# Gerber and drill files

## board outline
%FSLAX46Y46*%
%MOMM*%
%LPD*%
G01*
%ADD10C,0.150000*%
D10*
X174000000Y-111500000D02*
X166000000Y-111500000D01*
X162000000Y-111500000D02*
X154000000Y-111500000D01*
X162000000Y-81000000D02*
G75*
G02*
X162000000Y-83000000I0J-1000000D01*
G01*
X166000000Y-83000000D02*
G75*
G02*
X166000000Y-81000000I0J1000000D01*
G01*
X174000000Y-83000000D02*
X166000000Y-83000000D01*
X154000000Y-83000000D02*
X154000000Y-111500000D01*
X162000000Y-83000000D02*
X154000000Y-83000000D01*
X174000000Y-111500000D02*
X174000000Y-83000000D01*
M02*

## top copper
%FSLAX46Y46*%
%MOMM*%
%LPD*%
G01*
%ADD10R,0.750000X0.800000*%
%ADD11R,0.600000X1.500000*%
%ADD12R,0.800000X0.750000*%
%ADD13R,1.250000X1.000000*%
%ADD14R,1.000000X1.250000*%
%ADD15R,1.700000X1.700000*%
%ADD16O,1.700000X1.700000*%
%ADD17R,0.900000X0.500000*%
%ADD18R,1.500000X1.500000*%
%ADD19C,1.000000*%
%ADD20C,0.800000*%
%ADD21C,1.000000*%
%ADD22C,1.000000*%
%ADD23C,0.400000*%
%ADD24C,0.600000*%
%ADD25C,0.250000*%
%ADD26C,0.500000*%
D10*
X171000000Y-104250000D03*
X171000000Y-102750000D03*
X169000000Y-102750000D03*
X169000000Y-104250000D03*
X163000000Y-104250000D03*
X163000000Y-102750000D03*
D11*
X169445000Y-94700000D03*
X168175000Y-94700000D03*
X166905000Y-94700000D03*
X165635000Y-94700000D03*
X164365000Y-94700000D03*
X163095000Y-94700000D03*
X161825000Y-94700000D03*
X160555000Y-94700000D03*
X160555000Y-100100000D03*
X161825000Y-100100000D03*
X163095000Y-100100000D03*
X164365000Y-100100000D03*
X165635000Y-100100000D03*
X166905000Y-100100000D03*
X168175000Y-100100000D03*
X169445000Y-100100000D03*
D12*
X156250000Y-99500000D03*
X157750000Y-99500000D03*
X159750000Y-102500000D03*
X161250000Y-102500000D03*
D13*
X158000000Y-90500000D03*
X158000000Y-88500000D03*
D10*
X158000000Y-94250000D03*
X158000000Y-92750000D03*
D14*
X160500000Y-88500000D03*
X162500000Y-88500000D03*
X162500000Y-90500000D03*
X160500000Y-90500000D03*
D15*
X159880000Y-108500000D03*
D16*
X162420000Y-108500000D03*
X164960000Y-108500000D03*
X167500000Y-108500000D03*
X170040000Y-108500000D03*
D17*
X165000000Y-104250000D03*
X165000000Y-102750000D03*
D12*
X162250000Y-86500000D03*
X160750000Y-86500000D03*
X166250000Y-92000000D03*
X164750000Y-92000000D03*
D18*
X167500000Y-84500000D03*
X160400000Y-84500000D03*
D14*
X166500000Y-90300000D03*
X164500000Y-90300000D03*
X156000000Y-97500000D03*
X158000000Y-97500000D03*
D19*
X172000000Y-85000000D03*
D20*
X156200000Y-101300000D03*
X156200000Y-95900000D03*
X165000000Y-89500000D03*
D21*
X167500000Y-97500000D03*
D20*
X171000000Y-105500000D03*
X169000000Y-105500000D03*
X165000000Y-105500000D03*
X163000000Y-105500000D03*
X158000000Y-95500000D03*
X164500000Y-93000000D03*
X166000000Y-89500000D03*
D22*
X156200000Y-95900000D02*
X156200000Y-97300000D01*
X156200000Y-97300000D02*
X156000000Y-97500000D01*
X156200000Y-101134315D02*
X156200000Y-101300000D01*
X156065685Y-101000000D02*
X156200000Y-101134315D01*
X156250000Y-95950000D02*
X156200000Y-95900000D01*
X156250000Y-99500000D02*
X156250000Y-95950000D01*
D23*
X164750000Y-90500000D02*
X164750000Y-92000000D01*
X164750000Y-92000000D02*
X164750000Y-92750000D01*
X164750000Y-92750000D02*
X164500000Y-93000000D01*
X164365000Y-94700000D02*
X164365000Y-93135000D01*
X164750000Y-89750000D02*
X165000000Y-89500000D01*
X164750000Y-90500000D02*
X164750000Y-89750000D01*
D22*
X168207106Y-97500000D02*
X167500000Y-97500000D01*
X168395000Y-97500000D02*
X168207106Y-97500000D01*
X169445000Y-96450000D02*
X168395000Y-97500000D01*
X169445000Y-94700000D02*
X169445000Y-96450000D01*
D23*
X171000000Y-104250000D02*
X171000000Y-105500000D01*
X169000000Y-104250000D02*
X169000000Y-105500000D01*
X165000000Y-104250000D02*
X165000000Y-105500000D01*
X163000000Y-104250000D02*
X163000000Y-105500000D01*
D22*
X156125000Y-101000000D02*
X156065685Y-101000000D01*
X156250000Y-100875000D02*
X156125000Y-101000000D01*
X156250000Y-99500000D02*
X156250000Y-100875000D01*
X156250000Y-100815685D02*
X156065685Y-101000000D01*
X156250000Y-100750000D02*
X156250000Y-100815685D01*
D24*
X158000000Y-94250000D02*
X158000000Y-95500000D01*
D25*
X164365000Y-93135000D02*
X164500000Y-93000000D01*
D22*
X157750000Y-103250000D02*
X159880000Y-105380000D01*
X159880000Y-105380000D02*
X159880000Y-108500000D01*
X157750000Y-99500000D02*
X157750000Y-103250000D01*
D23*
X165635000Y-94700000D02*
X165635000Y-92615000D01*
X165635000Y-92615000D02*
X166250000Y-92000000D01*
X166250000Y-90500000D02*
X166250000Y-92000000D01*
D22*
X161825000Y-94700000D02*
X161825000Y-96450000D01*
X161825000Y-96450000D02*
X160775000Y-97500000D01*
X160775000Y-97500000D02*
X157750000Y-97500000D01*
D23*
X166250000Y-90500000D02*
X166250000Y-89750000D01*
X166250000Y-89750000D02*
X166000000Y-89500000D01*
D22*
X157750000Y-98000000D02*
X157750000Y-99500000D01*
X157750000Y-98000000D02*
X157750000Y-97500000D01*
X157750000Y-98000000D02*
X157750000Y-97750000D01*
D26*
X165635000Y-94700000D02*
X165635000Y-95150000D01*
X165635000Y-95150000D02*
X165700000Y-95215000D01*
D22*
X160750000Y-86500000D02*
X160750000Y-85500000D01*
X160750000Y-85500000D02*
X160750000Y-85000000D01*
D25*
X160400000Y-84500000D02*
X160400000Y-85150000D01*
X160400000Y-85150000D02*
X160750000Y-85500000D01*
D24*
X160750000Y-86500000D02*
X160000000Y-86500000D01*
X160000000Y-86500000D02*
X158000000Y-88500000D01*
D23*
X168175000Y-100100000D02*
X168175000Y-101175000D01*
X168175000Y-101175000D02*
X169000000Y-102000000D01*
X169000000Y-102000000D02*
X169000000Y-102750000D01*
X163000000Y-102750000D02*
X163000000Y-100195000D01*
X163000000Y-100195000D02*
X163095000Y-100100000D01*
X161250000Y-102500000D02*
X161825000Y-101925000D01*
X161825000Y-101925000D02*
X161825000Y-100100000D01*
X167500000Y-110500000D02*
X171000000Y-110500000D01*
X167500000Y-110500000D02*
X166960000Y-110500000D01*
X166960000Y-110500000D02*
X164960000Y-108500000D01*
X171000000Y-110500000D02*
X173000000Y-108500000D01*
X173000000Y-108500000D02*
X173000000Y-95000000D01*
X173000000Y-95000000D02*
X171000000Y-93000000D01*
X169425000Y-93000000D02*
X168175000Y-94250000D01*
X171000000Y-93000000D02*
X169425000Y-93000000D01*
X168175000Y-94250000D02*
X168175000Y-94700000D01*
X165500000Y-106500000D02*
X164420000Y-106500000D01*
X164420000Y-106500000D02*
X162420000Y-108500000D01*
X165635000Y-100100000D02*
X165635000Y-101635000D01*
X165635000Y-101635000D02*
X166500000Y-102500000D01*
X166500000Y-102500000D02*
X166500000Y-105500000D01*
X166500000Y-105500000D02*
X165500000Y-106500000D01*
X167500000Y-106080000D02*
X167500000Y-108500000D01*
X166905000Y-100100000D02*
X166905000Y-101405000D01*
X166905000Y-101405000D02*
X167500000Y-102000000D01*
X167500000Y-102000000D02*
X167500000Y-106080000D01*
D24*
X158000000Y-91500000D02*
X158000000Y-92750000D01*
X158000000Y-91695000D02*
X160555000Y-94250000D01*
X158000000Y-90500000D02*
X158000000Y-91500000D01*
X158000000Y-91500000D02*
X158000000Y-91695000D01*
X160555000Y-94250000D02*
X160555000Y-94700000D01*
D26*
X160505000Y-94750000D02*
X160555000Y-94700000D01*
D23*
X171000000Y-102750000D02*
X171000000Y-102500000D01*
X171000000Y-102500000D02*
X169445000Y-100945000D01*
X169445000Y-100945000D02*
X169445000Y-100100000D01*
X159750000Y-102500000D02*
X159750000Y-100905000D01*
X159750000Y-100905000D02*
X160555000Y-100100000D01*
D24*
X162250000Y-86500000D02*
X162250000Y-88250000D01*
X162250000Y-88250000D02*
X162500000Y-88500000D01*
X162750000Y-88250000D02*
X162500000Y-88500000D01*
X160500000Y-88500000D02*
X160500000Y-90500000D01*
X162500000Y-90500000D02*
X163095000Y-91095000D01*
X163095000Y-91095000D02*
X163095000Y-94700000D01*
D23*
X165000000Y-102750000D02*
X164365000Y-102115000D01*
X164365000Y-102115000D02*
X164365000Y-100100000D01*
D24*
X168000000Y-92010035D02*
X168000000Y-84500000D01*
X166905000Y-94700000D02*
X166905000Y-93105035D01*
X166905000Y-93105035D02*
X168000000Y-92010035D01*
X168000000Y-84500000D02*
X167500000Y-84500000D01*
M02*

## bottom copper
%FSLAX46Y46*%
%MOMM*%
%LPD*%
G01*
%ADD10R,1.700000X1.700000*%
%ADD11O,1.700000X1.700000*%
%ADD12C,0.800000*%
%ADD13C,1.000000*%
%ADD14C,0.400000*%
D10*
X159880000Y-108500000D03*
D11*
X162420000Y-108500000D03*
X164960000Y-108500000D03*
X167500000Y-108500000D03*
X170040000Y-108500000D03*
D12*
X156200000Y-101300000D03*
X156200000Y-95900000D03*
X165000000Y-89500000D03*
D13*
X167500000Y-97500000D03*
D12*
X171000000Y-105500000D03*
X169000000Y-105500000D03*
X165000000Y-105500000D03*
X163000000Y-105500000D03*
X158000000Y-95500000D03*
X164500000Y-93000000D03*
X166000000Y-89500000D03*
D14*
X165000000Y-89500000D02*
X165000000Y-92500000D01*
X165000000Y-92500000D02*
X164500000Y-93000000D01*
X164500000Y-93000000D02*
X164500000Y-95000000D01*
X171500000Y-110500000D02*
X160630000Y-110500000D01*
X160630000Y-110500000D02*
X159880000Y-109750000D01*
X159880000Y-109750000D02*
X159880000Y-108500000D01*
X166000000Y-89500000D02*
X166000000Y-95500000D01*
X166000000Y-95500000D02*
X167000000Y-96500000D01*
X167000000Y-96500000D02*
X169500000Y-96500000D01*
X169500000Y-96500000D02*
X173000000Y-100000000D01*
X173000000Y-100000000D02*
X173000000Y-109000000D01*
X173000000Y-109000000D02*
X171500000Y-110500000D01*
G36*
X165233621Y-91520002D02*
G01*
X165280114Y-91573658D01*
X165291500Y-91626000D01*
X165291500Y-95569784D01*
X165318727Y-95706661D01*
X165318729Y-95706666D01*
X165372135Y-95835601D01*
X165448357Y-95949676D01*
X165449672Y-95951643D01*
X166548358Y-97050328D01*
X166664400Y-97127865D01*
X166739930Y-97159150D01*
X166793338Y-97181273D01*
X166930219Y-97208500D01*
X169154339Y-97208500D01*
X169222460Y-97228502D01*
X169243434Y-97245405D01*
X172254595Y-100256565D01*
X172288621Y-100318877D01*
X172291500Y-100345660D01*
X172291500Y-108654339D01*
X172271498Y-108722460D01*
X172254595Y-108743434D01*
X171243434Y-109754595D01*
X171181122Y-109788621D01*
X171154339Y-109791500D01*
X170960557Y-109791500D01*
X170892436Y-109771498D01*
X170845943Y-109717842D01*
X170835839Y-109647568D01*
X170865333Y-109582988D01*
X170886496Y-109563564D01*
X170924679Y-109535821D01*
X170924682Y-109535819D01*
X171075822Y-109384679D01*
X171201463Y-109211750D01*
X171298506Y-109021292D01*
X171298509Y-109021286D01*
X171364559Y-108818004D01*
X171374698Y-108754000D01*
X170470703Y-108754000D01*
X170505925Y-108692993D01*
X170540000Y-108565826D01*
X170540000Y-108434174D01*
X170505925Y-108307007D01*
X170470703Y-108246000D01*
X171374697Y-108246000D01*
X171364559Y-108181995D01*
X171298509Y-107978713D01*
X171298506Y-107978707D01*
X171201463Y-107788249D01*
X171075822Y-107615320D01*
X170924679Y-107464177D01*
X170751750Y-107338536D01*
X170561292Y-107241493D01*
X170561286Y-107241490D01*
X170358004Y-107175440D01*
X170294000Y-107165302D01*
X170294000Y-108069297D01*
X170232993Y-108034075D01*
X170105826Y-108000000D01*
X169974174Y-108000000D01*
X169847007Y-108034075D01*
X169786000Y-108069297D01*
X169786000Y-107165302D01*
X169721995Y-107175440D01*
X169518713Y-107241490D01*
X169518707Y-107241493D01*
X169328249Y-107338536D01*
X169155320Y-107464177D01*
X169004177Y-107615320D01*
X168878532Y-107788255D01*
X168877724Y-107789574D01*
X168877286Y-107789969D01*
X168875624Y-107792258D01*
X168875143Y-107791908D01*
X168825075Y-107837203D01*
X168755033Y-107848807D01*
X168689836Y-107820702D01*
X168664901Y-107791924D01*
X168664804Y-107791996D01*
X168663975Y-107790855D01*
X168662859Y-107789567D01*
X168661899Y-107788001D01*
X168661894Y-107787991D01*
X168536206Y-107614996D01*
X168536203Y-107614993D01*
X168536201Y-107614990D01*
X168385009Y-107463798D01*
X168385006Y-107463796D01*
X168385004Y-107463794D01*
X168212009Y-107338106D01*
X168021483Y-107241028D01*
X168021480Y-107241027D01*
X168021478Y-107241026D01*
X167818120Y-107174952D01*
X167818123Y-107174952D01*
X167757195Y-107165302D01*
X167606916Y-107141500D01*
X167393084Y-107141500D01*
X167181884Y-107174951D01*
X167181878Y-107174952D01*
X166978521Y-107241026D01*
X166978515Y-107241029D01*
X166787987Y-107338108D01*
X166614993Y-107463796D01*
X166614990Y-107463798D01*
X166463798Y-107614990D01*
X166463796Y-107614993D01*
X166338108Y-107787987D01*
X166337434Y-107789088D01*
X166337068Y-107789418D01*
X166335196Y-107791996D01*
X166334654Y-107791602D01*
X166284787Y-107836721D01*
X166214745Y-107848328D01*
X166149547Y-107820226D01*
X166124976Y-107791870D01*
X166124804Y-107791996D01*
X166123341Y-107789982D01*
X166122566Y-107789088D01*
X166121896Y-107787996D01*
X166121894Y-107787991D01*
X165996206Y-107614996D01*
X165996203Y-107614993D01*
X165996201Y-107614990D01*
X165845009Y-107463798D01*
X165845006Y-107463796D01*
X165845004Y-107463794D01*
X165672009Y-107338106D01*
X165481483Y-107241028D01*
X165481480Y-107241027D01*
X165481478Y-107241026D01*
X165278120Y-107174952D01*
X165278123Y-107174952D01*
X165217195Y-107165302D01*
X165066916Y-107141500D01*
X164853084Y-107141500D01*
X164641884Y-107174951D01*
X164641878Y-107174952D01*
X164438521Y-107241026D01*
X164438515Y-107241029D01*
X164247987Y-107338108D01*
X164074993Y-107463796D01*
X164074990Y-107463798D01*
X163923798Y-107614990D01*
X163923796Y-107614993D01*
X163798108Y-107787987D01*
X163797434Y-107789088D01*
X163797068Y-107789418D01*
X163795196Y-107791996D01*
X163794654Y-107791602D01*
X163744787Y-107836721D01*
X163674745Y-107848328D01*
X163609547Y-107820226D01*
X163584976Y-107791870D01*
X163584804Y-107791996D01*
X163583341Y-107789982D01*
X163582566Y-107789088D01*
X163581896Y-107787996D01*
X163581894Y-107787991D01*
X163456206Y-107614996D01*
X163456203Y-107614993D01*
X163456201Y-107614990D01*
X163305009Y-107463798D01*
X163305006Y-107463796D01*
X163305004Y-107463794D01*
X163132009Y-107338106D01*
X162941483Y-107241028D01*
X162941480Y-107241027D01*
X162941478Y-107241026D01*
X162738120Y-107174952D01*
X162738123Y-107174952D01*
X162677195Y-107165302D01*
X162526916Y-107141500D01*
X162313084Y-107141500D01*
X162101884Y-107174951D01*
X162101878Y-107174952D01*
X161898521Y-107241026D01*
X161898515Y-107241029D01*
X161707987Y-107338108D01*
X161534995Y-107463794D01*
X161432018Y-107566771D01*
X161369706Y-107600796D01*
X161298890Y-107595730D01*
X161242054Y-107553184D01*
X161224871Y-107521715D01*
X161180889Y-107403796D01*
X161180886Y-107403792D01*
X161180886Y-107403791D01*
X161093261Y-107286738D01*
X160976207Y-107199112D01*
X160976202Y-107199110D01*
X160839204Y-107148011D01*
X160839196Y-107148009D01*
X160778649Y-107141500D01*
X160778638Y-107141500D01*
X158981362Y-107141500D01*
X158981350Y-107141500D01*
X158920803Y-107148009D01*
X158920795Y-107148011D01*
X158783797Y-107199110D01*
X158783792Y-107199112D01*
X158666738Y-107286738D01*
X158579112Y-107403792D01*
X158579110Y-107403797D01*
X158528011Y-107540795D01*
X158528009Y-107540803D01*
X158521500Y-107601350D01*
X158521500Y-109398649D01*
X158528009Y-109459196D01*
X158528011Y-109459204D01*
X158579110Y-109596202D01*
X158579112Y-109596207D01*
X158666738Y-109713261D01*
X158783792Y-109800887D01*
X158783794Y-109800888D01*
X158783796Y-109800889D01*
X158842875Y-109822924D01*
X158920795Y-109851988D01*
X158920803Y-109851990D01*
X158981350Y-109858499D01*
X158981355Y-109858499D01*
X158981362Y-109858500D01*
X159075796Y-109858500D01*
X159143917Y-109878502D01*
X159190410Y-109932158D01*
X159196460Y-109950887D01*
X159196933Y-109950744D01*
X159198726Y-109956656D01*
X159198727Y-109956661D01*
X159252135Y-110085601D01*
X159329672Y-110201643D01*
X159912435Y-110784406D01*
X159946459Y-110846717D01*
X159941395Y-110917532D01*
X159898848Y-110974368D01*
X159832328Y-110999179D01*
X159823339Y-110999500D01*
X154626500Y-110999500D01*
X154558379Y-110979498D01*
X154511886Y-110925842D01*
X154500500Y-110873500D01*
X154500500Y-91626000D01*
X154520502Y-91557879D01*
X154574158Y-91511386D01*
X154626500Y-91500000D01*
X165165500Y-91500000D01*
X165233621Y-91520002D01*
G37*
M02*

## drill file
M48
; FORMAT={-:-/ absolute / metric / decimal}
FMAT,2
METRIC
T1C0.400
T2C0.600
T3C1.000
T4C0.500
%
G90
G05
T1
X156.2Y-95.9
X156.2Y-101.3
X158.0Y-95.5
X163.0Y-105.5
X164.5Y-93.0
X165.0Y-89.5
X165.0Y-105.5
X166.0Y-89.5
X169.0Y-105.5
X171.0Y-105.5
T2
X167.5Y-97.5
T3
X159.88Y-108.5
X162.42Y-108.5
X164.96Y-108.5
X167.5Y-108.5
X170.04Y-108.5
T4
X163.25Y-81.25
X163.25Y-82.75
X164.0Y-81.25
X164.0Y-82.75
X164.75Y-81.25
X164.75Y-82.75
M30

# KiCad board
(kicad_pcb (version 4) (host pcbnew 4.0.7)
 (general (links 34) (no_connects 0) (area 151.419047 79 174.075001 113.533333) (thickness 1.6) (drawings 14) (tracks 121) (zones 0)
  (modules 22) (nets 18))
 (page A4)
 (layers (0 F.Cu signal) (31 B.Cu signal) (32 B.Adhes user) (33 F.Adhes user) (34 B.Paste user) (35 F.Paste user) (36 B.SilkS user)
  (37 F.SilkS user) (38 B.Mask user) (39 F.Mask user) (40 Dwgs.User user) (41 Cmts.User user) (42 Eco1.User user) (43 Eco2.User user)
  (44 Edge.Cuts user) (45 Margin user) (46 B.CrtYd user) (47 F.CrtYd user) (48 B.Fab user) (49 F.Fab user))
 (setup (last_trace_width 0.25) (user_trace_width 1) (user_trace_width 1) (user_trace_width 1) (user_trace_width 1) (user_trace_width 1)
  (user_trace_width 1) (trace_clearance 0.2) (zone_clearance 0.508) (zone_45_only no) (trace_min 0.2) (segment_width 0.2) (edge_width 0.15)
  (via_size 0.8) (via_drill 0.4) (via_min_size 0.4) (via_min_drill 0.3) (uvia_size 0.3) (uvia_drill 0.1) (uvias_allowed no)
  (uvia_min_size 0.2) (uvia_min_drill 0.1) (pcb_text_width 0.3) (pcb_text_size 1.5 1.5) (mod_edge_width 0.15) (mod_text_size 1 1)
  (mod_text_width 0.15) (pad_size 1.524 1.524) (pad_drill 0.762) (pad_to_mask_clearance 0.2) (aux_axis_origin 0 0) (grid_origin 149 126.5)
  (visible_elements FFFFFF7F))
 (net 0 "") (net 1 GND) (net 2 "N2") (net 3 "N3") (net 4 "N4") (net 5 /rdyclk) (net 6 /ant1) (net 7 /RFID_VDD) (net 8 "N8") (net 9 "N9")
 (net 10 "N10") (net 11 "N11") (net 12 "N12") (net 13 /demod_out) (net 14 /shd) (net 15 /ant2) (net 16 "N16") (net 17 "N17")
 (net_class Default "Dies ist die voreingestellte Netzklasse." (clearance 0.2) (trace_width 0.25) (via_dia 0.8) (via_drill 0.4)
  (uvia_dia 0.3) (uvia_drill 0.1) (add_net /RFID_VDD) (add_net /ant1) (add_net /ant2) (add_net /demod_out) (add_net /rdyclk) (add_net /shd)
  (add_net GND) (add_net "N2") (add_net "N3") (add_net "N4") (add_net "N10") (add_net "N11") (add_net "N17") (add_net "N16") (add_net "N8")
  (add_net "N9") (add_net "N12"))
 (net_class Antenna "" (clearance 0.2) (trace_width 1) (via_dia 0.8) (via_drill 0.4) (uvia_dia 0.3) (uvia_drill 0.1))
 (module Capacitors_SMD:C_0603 (layer F.Cu) (at 171 103.5 90)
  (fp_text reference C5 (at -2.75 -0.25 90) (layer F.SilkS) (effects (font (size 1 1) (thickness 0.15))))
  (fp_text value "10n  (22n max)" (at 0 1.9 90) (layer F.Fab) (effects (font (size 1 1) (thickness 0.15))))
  (pad 1 smd rect (at -0.75 0 90) (size 0.8 0.75) (layers F.Cu F.Paste F.Mask) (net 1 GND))
  (pad 2 smd rect (at 0.75 0 90) (size 0.8 0.75) (layers F.Cu F.Paste F.Mask) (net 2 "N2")))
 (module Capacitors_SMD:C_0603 (layer F.Cu) (at 169 103.5 90)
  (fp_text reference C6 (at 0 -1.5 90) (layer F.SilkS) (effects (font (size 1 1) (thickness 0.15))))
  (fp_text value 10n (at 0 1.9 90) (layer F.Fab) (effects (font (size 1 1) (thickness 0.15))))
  (pad 2 smd rect (at 0.75 0 90) (size 0.8 0.75) (layers F.Cu F.Paste F.Mask) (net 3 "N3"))
  (pad 1 smd rect (at -0.75 0 90) (size 0.8 0.75) (layers F.Cu F.Paste F.Mask) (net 1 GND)))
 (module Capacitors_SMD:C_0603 (layer F.Cu) (at 163 103.5 90)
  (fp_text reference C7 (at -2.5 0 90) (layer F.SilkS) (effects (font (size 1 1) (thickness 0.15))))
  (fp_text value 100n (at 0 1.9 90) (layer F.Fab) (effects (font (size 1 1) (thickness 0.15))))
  (pad 1 smd rect (at -0.75 0 90) (size 0.8 0.75) (layers F.Cu F.Paste F.Mask) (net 1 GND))
  (pad 2 smd rect (at 0.75 0 90) (size 0.8 0.75) (layers F.Cu F.Paste F.Mask) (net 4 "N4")))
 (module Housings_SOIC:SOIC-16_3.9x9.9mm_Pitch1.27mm (layer F.Cu) (at 165 97.4 270)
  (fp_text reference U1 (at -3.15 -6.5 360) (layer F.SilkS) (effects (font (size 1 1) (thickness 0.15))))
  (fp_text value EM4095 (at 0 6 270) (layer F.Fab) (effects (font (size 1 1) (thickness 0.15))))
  (pad 1 smd rect (at -2.7 -4.445 270) (size 1.5 0.6) (layers F.Cu F.Paste F.Mask) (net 1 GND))
  (pad 2 smd rect (at -2.7 -3.175 270) (size 1.5 0.6) (layers F.Cu F.Paste F.Mask) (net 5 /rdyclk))
  (pad 3 smd rect (at -2.7 -1.905 270) (size 1.5 0.6) (layers F.Cu F.Paste F.Mask) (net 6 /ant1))
  (pad 4 smd rect (at -2.7 -0.635 270) (size 1.5 0.6) (layers F.Cu F.Paste F.Mask) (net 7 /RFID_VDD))
  (pad 5 smd rect (at -2.7 0.635 270) (size 1.5 0.6) (layers F.Cu F.Paste F.Mask) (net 1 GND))
  (pad 6 smd rect (at -2.7 1.905 270) (size 1.5 0.6) (layers F.Cu F.Paste F.Mask) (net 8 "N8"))
  (pad 7 smd rect (at -2.7 3.175 270) (size 1.5 0.6) (layers F.Cu F.Paste F.Mask) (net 7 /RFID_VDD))
  (pad 8 smd rect (at -2.7 4.445 270) (size 1.5 0.6) (layers F.Cu F.Paste F.Mask) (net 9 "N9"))
  (pad 9 smd rect (at 2.7 4.445 270) (size 1.5 0.6) (layers F.Cu F.Paste F.Mask) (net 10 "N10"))
  (pad 10 smd rect (at 2.7 3.175 270) (size 1.5 0.6) (layers F.Cu F.Paste F.Mask) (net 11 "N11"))
  (pad 11 smd rect (at 2.7 1.905 270) (size 1.5 0.6) (layers F.Cu F.Paste F.Mask) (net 4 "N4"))
  (pad 12 smd rect (at 2.7 0.635 270) (size 1.5 0.6) (layers F.Cu F.Paste F.Mask) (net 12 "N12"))
  (pad 13 smd rect (at 2.7 -0.635 270) (size 1.5 0.6) (layers F.Cu F.Paste F.Mask) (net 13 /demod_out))
  (pad 14 smd rect (at 2.7 -1.905 270) (size 1.5 0.6) (layers F.Cu F.Paste F.Mask) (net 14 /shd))
  (pad 15 smd rect (at 2.7 -3.175 270) (size 1.5 0.6) (layers F.Cu F.Paste F.Mask) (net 3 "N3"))
  (pad 16 smd rect (at 2.7 -4.445 270) (size 1.5 0.6) (layers F.Cu F.Paste F.Mask) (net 2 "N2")))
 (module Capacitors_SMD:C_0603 (layer F.Cu) (at 157 99.5)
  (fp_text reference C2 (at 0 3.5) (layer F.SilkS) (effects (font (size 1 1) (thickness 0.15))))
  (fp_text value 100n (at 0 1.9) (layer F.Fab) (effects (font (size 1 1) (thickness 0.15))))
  (pad 1 smd rect (at -0.75 0) (size 0.8 0.75) (layers F.Cu F.Paste F.Mask) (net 1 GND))
  (pad 2 smd rect (at 0.75 0) (size 0.8 0.75) (layers F.Cu F.Paste F.Mask) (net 7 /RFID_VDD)))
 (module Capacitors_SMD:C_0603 (layer F.Cu) (at 160.5 102.5)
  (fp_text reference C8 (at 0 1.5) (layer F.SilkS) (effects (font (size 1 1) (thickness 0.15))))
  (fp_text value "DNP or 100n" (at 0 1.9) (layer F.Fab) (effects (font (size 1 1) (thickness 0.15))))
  (pad 1 smd rect (at -0.75 0) (size 0.8 0.75) (layers F.Cu F.Paste F.Mask) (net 10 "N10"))
  (pad 2 smd rect (at 0.75 0) (size 0.8 0.75) (layers F.Cu F.Paste F.Mask) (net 11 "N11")))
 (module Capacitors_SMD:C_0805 (layer F.Cu) (at 158 89.5 90)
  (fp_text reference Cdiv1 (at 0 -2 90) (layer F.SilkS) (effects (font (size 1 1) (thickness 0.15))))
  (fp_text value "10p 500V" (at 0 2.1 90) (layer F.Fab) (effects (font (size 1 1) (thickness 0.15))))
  (pad 1 smd rect (at -1 0 90) (size 1 1.25) (layers F.Cu F.Paste F.Mask) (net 9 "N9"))
  (pad 2 smd rect (at 1 0 90) (size 1 1.25) (layers F.Cu F.Paste F.Mask) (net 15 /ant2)))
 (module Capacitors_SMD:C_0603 (layer F.Cu) (at 158 93.5 90)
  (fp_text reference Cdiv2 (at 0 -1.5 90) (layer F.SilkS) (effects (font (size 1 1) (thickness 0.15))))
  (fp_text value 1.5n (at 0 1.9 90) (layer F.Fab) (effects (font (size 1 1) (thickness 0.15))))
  (pad 1 smd rect (at -0.75 0 90) (size 0.8 0.75) (layers F.Cu F.Paste F.Mask) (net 1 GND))
  (pad 2 smd rect (at 0.75 0 90) (size 0.8 0.75) (layers F.Cu F.Paste F.Mask) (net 9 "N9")))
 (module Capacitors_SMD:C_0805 (layer F.Cu) (at 161.5 88.5)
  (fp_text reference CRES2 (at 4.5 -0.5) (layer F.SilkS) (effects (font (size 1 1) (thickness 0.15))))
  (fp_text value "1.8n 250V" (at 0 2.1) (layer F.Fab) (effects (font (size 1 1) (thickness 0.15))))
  (pad 1 smd rect (at -1 0) (size 1 1.25) (layers F.Cu F.Paste F.Mask) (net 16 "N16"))
  (pad 2 smd rect (at 1 0) (size 1 1.25) (layers F.Cu F.Paste F.Mask) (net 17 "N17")))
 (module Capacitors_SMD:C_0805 (layer F.Cu) (at 161.5 90.5 180)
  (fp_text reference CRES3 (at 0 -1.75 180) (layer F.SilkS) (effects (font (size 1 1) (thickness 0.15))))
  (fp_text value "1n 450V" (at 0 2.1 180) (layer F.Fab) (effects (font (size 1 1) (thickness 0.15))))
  (pad 1 smd rect (at -1 0 180) (size 1 1.25) (layers F.Cu F.Paste F.Mask) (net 8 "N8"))
  (pad 2 smd rect (at 1 0 180) (size 1 1.25) (layers F.Cu F.Paste F.Mask) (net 16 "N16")))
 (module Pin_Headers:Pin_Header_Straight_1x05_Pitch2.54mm (layer F.Cu) (at 159.88 108.5 90)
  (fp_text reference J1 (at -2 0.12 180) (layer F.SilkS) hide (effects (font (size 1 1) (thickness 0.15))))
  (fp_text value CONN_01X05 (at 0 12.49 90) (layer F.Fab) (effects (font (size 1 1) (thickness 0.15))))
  (pad 1 thru_hole rect (at 0 0 90) (size 1.7 1.7) (drill 1) (layers *.Cu *.Mask) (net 7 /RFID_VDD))
  (pad 2 thru_hole oval (at 0 2.54 90) (size 1.7 1.7) (drill 1) (layers *.Cu *.Mask) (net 13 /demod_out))
  (pad 3 thru_hole oval (at 0 5.08 90) (size 1.7 1.7) (drill 1) (layers *.Cu *.Mask) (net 5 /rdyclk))
  (pad 4 thru_hole oval (at 0 7.62 90) (size 1.7 1.7) (drill 1) (layers *.Cu *.Mask) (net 14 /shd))
  (pad 5 thru_hole oval (at 0 10.16 90) (size 1.7 1.7) (drill 1) (layers *.Cu *.Mask) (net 1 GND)))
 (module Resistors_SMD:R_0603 (layer F.Cu) (at 165 103.5 90)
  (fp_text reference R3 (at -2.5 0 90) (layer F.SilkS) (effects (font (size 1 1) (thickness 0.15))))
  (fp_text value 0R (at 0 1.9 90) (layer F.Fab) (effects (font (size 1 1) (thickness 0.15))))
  (pad 1 smd rect (at -0.75 0 90) (size 0.5 0.9) (layers F.Cu F.Paste F.Mask) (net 1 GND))
  (pad 2 smd rect (at 0.75 0 90) (size 0.5 0.9) (layers F.Cu F.Paste F.Mask) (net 12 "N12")))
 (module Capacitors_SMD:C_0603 (layer F.Cu) (at 161.5 86.5 180)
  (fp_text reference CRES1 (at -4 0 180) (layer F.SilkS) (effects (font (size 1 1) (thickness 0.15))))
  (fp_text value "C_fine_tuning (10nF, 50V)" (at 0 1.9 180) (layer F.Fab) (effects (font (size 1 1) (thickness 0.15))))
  (pad 1 smd rect (at -0.75 0 180) (size 0.8 0.75) (layers F.Cu F.Paste F.Mask) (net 17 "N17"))
  (pad 2 smd rect (at 0.75 0 180) (size 0.8 0.75) (layers F.Cu F.Paste F.Mask) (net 15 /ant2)))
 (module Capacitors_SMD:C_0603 (layer F.Cu) (at 165.5 92 180)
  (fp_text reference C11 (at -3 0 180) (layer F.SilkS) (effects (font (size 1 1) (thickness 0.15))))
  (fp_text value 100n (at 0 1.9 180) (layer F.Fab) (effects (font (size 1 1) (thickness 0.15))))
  (pad 1 smd rect (at -0.75 0 180) (size 0.8 0.75) (layers F.Cu F.Paste F.Mask) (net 7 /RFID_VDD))
  (pad 2 smd rect (at 0.75 0 180) (size 0.8 0.75) (layers F.Cu F.Paste F.Mask) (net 1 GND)))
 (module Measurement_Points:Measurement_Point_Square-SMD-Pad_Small (layer F.Cu) (at 167.5 84.5)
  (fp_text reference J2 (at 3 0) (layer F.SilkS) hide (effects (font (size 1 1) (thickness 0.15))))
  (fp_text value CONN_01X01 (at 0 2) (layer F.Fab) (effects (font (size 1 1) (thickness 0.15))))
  (pad 1 smd rect (at 0 0) (size 1.5 1.5) (layers F.Cu F.Mask) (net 6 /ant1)))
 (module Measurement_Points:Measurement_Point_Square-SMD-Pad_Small (layer F.Cu) (at 160.4 84.5)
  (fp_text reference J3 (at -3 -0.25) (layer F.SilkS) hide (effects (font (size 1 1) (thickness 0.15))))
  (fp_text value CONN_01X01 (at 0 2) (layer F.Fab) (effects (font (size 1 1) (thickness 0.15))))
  (pad 1 smd rect (at 0 0) (size 1.5 1.5) (layers F.Cu F.Mask) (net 15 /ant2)))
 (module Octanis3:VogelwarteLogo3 (layer B.Cu) (at 164 104 180)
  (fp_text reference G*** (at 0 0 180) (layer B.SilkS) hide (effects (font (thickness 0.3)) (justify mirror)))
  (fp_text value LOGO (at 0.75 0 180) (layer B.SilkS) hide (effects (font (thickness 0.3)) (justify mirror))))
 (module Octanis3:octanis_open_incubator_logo (layer B.Cu) (at 164 91.5 180)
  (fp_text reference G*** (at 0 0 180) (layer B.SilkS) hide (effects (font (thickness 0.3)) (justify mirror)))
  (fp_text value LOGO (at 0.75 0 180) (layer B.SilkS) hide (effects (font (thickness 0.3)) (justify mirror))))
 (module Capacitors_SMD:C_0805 (layer F.Cu) (at 165.5 90.3 180)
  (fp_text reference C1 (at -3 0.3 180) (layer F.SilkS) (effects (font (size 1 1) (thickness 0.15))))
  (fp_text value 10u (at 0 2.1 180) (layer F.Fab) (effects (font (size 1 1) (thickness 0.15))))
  (pad 1 smd rect (at -1 0 180) (size 1 1.25) (layers F.Cu F.Paste F.Mask) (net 7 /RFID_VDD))
  (pad 2 smd rect (at 1 0 180) (size 1 1.25) (layers F.Cu F.Paste F.Mask) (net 1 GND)))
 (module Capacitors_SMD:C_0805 (layer F.Cu) (at 157 97.5)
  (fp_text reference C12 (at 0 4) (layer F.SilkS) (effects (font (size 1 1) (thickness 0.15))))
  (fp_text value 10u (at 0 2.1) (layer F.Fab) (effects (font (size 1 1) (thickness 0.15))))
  (pad 1 smd rect (at -1 0) (size 1 1.25) (layers F.Cu F.Paste F.Mask) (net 1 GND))
  (pad 2 smd rect (at 1 0) (size 1 1.25) (layers F.Cu F.Paste F.Mask) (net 7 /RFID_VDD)))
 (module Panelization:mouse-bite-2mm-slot (layer F.Cu) (at 164 82)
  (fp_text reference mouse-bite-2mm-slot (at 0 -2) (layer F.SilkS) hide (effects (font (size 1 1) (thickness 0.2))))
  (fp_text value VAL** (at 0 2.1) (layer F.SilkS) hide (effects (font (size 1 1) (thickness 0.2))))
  (pad "" np_thru_hole circle (at 0 -0.75) (size 0.5 0.5) (drill 0.5) (layers *.Cu *.Mask))
  (pad "" np_thru_hole circle (at 0 0.75) (size 0.5 0.5) (drill 0.5) (layers *.Cu *.Mask))
  (pad "" np_thru_hole circle (at 0.75 -0.75) (size 0.5 0.5) (drill 0.5) (layers *.Cu *.Mask))
  (pad "" np_thru_hole circle (at -0.75 -0.75) (size 0.5 0.5) (drill 0.5) (layers *.Cu *.Mask))
  (pad "" np_thru_hole circle (at -0.75 0.75) (size 0.5 0.5) (drill 0.5) (layers *.Cu *.Mask))
  (pad "" np_thru_hole circle (at 0.75 0.75) (size 0.5 0.5) (drill 0.5) (layers *.Cu *.Mask)))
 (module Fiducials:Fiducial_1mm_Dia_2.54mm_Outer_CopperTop (layer F.Cu) (at 172 85)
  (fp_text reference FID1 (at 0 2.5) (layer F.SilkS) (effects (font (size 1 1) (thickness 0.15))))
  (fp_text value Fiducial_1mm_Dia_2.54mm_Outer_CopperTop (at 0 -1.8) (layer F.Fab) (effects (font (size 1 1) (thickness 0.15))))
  (pad ~ smd circle (at 0 0) (size 1 1) (layers F.Cu F.Mask) (solder_mask_margin 0.77) (clearance 0.77)))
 (gr_line (start 174 111.5) (end 166 111.5) (layer Edge.Cuts) (width 0.15))
 (gr_line (start 162 111.5) (end 154 111.5) (layer Edge.Cuts) (width 0.15))
 (gr_arc (start 162 82) (end 162 81) (angle 180) (layer Edge.Cuts) (width 0.15))
 (gr_arc (start 166 82) (end 166 83) (angle 180) (layer Edge.Cuts) (width 0.15))
 (gr_line (start 174 83) (end 166 83) (layer Edge.Cuts) (width 0.15))
 (gr_line (start 154 83) (end 154 111.5) (layer Edge.Cuts) (width 0.15))
 (gr_line (start 162 83) (end 154 83) (layer Edge.Cuts) (width 0.15))
 (gr_line (start 174 111.5) (end 174 83) (layer Edge.Cuts) (width 0.15))
 (segment (start 156.2 95.9) (end 156.2 97.3) (width 1) (layer F.Cu) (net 1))
 (segment (start 156.2 97.3) (end 156 97.5) (width 1) (layer F.Cu) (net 1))
 (segment (start 156.2 101.134315) (end 156.2 101.3) (width 1) (layer F.Cu) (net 1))
 (segment (start 156.065685 101) (end 156.2 101.134315) (width 1) (layer F.Cu) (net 1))
 (via (at 156.2 101.3) (size 0.8) (drill 0.4) (layers F.Cu B.Cu) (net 1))
 (segment (start 156.25 95.95) (end 156.2 95.9) (width 1) (layer F.Cu) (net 1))
 (segment (start 156.25 99.5) (end 156.25 95.95) (width 1) (layer F.Cu) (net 1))
 (via (at 156.2 95.9) (size 0.8) (drill 0.4) (layers F.Cu B.Cu) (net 1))
 (segment (start 164.75 90.5) (end 164.75 92) (width 0.4) (layer F.Cu) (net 1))
 (segment (start 164.75 92) (end 164.75 92.75) (width 0.4) (layer F.Cu) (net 1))
 (segment (start 164.75 92.75) (end 164.5 93) (width 0.4) (layer F.Cu) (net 1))
 (segment (start 164.365 94.7) (end 164.365 93.135) (width 0.4) (layer F.Cu) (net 1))
 (segment (start 164.75 89.75) (end 165 89.5) (width 0.4) (layer F.Cu) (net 1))
 (segment (start 164.75 90.5) (end 164.75 89.75) (width 0.4) (layer F.Cu) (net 1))
 (segment (start 165 89.5) (end 165 92.5) (width 0.4) (layer B.Cu) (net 1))
 (segment (start 165 92.5) (end 164.5 93) (width 0.4) (layer B.Cu) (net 1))
 (via (at 165 89.5) (size 0.8) (drill 0.4) (layers F.Cu B.Cu) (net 1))
 (segment (start 164.5 93) (end 164.5 95) (width 0.4) (layer B.Cu) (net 1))
 (segment (start 168.207106 97.5) (end 167.5 97.5) (width 1) (layer F.Cu) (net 1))
 (segment (start 168.395 97.5) (end 168.207106 97.5) (width 1) (layer F.Cu) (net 1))
 (segment (start 169.445 96.45) (end 168.395 97.5) (width 1) (layer F.Cu) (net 1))
 (segment (start 169.445 94.7) (end 169.445 96.45) (width 1) (layer F.Cu) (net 1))
 (via (at 167.5 97.5) (size 1) (drill 0.6) (layers F.Cu B.Cu) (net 1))
 (segment (start 171 104.25) (end 171 105.5) (width 0.4) (layer F.Cu) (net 1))
 (via (at 171 105.5) (size 0.8) (drill 0.4) (layers F.Cu B.Cu) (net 1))
 (segment (start 169 104.25) (end 169 105.5) (width 0.4) (layer F.Cu) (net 1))
 (via (at 169 105.5) (size 0.8) (drill 0.4) (layers F.Cu B.Cu) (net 1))
 (segment (start 165 104.25) (end 165 105.5) (width 0.4) (layer F.Cu) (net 1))
 (via (at 165 105.5) (size 0.8) (drill 0.4) (layers F.Cu B.Cu) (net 1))
 (segment (start 163 104.25) (end 163 105.5) (width 0.4) (layer F.Cu) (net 1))
 (via (at 163 105.5) (size 0.8) (drill 0.4) (layers F.Cu B.Cu) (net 1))
 (segment (start 156.125 101) (end 156.065685 101) (width 1) (layer F.Cu) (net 1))
 (segment (start 156.25 100.875) (end 156.125 101) (width 1) (layer F.Cu) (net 1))
 (segment (start 156.25 99.5) (end 156.25 100.875) (width 1) (layer F.Cu) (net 1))
 (segment (start 156.25 100.815685) (end 156.065685 101) (width 1) (layer F.Cu) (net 1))
 (segment (start 156.25 100.75) (end 156.25 100.815685) (width 1) (layer F.Cu) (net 1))
 (segment (start 158 94.25) (end 158 95.5) (width 0.6) (layer F.Cu) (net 1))
 (via (at 158 95.5) (size 0.8) (drill 0.4) (layers F.Cu B.Cu) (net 1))
 (via (at 164.5 93) (size 0.8) (drill 0.4) (layers F.Cu B.Cu) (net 1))
 (segment (start 164.365 93.135) (end 164.5 93) (width 0.25) (layer F.Cu) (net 1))
 (segment (start 171.5 110.5) (end 160.63 110.5) (width 0.4) (layer B.Cu) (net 7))
 (segment (start 160.63 110.5) (end 159.88 109.75) (width 0.4) (layer B.Cu) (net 7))
 (segment (start 159.88 109.75) (end 159.88 108.5) (width 0.4) (layer B.Cu) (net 7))
 (segment (start 157.75 103.25) (end 159.88 105.38) (width 1) (layer F.Cu) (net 7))
 (segment (start 159.88 105.38) (end 159.88 108.5) (width 1) (layer F.Cu) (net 7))
 (segment (start 157.75 99.5) (end 157.75 103.25) (width 1) (layer F.Cu) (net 7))
 (segment (start 166 89.5) (end 166 95.5) (width 0.4) (layer B.Cu) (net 7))
 (segment (start 166 95.5) (end 167 96.5) (width 0.4) (layer B.Cu) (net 7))
 (segment (start 167 96.5) (end 169.5 96.5) (width 0.4) (layer B.Cu) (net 7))
 (segment (start 169.5 96.5) (end 173 100) (width 0.4) (layer B.Cu) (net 7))
 (segment (start 173 100) (end 173 109) (width 0.4) (layer B.Cu) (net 7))
 (segment (start 173 109) (end 171.5 110.5) (width 0.4) (layer B.Cu) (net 7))
 (segment (start 165.635 94.7) (end 165.635 92.615) (width 0.4) (layer F.Cu) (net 7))
 (segment (start 165.635 92.615) (end 166.25 92) (width 0.4) (layer F.Cu) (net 7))
 (segment (start 166.25 90.5) (end 166.25 92) (width 0.4) (layer F.Cu) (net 7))
 (segment (start 161.825 94.7) (end 161.825 96.45) (width 1) (layer F.Cu) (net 7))
 (segment (start 161.825 96.45) (end 160.775 97.5) (width 1) (layer F.Cu) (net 7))
 (segment (start 160.775 97.5) (end 157.75 97.5) (width 1) (layer F.Cu) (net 7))
 (segment (start 166.25 90.5) (end 166.25 89.75) (width 0.4) (layer F.Cu) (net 7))
 (segment (start 166.25 89.75) (end 166 89.5) (width 0.4) (layer F.Cu) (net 7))
 (via (at 166 89.5) (size 0.8) (drill 0.4) (layers F.Cu B.Cu) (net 7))
 (segment (start 157.75 98) (end 157.75 99.5) (width 1) (layer F.Cu) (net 7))
 (segment (start 157.75 98) (end 157.75 97.5) (width 1) (layer F.Cu) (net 7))
 (segment (start 157.75 98) (end 157.75 97.75) (width 1) (layer F.Cu) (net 7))
 (segment (start 165.635 94.7) (end 165.635 95.15) (width 0.5) (layer F.Cu) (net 7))
 (segment (start 165.635 95.15) (end 165.7 95.215) (width 0.5) (layer F.Cu) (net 7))
 (segment (start 160.75 86.5) (end 160.75 85.5) (width 1) (layer F.Cu) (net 15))
 (segment (start 160.75 85.5) (end 160.75 85) (width 1) (layer F.Cu) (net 15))
 (segment (start 160.4 84.5) (end 160.4 85.15) (width 0.25) (layer F.Cu) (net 15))
 (segment (start 160.4 85.15) (end 160.75 85.5) (width 0.25) (layer F.Cu) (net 15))
 (segment (start 160.75 86.5) (end 160 86.5) (width 0.6) (layer F.Cu) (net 15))
 (segment (start 160 86.5) (end 158 88.5) (width 0.6) (layer F.Cu) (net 15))
 (segment (start 168.175 100.1) (end 168.175 101.175) (width 0.4) (layer F.Cu) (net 3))
 (segment (start 168.175 101.175) (end 169 102) (width 0.4) (layer F.Cu) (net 3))
 (segment (start 169 102) (end 169 102.75) (width 0.4) (layer F.Cu) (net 3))
 (segment (start 163 102.75) (end 163 100.195) (width 0.4) (layer F.Cu) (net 4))
 (segment (start 163 100.195) (end 163.095 100.1) (width 0.4) (layer F.Cu) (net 4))
 (segment (start 161.25 102.5) (end 161.825 101.925) (width 0.4) (layer F.Cu) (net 11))
 (segment (start 161.825 101.925) (end 161.825 100.1) (width 0.4) (layer F.Cu) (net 11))
 (segment (start 167.5 110.5) (end 171 110.5) (width 0.4) (layer F.Cu) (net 5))
 (segment (start 167.5 110.5) (end 166.96 110.5) (width 0.4) (layer F.Cu) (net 5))
 (segment (start 166.96 110.5) (end 164.96 108.5) (width 0.4) (layer F.Cu) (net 5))
 (segment (start 171 110.5) (end 173 108.5) (width 0.4) (layer F.Cu) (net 5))
 (segment (start 173 108.5) (end 173 95) (width 0.4) (layer F.Cu) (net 5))
 (segment (start 173 95) (end 171 93) (width 0.4) (layer F.Cu) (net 5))
 (segment (start 169.425 93) (end 168.175 94.25) (width 0.4) (layer F.Cu) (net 5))
 (segment (start 171 93) (end 169.425 93) (width 0.4) (layer F.Cu) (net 5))
 (segment (start 168.175 94.25) (end 168.175 94.7) (width 0.4) (layer F.Cu) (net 5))
 (segment (start 165.5 106.5) (end 164.42 106.5) (width 0.4) (layer F.Cu) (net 13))
 (segment (start 164.42 106.5) (end 162.42 108.5) (width 0.4) (layer F.Cu) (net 13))
 (segment (start 165.635 100.1) (end 165.635 101.635) (width 0.4) (layer F.Cu) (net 13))
 (segment (start 165.635 101.635) (end 166.5 102.5) (width 0.4) (layer F.Cu) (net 13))
 (segment (start 166.5 102.5) (end 166.5 105.5) (width 0.4) (layer F.Cu) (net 13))
 (segment (start 166.5 105.5) (end 165.5 106.5) (width 0.4) (layer F.Cu) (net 13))
 (segment (start 167.5 106.08) (end 167.5 108.5) (width 0.4) (layer F.Cu) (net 14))
 (segment (start 166.905 100.1) (end 166.905 101.405) (width 0.4) (layer F.Cu) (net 14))
 (segment (start 166.905 101.405) (end 167.5 102) (width 0.4) (layer F.Cu) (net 14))
 (segment (start 167.5 102) (end 167.5 106.08) (width 0.4) (layer F.Cu) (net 14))
 (segment (start 158 91.5) (end 158 92.75) (width 0.6) (layer F.Cu) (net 9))
 (segment (start 158 91.695) (end 160.555 94.25) (width 0.6) (layer F.Cu) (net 9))
 (segment (start 158 90.5) (end 158 91.5) (width 0.6) (layer F.Cu) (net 9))
 (segment (start 158 91.5) (end 158 91.695) (width 0.6) (layer F.Cu) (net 9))
 (segment (start 160.555 94.25) (end 160.555 94.7) (width 0.6) (layer F.Cu) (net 9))
 (segment (start 160.505 94.75) (end 160.555 94.7) (width 0.5) (layer F.Cu) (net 9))
 (segment (start 171 102.75) (end 171 102.5) (width 0.4) (layer F.Cu) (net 2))
 (segment (start 171 102.5) (end 169.445 100.945) (width 0.4) (layer F.Cu) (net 2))
 (segment (start 169.445 100.945) (end 169.445 100.1) (width 0.4) (layer F.Cu) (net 2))
 (segment (start 159.75 102.5) (end 159.75 100.905) (width 0.4) (layer F.Cu) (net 10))
 (segment (start 159.75 100.905) (end 160.555 100.1) (width 0.4) (layer F.Cu) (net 10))
 (segment (start 162.25 86.5) (end 162.25 88.25) (width 0.6) (layer F.Cu) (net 17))
 (segment (start 162.25 88.25) (end 162.5 88.5) (width 0.6) (layer F.Cu) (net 17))
 (segment (start 162.75 88.25) (end 162.5 88.5) (width 0.6) (layer F.Cu) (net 17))
 (segment (start 160.5 88.5) (end 160.5 90.5) (width 0.6) (layer F.Cu) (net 16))
 (segment (start 162.5 90.5) (end 163.095 91.095) (width 0.6) (layer F.Cu) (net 8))
 (segment (start 163.095 91.095) (end 163.095 94.7) (width 0.6) (layer F.Cu) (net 8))
 (segment (start 165 102.75) (end 164.365 102.115) (width 0.4) (layer F.Cu) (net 12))
 (segment (start 164.365 102.115) (end 164.365 100.1) (width 0.4) (layer F.Cu) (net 12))
 (segment (start 168 92.010035) (end 168 84.5) (width 0.6) (layer F.Cu) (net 6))
 (segment (start 166.905 94.7) (end 166.905 93.105035) (width 0.6) (layer F.Cu) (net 6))
 (segment (start 166.905 93.105035) (end 168 92.010035) (width 0.6) (layer F.Cu) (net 6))
 (segment (start 168 84.5) (end 167.5 84.5) (width 0.6) (layer F.Cu) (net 6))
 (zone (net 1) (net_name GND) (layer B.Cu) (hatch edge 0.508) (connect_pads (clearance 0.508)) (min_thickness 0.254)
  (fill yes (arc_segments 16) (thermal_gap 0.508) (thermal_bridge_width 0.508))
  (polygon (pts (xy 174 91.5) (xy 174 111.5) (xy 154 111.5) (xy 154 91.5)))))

